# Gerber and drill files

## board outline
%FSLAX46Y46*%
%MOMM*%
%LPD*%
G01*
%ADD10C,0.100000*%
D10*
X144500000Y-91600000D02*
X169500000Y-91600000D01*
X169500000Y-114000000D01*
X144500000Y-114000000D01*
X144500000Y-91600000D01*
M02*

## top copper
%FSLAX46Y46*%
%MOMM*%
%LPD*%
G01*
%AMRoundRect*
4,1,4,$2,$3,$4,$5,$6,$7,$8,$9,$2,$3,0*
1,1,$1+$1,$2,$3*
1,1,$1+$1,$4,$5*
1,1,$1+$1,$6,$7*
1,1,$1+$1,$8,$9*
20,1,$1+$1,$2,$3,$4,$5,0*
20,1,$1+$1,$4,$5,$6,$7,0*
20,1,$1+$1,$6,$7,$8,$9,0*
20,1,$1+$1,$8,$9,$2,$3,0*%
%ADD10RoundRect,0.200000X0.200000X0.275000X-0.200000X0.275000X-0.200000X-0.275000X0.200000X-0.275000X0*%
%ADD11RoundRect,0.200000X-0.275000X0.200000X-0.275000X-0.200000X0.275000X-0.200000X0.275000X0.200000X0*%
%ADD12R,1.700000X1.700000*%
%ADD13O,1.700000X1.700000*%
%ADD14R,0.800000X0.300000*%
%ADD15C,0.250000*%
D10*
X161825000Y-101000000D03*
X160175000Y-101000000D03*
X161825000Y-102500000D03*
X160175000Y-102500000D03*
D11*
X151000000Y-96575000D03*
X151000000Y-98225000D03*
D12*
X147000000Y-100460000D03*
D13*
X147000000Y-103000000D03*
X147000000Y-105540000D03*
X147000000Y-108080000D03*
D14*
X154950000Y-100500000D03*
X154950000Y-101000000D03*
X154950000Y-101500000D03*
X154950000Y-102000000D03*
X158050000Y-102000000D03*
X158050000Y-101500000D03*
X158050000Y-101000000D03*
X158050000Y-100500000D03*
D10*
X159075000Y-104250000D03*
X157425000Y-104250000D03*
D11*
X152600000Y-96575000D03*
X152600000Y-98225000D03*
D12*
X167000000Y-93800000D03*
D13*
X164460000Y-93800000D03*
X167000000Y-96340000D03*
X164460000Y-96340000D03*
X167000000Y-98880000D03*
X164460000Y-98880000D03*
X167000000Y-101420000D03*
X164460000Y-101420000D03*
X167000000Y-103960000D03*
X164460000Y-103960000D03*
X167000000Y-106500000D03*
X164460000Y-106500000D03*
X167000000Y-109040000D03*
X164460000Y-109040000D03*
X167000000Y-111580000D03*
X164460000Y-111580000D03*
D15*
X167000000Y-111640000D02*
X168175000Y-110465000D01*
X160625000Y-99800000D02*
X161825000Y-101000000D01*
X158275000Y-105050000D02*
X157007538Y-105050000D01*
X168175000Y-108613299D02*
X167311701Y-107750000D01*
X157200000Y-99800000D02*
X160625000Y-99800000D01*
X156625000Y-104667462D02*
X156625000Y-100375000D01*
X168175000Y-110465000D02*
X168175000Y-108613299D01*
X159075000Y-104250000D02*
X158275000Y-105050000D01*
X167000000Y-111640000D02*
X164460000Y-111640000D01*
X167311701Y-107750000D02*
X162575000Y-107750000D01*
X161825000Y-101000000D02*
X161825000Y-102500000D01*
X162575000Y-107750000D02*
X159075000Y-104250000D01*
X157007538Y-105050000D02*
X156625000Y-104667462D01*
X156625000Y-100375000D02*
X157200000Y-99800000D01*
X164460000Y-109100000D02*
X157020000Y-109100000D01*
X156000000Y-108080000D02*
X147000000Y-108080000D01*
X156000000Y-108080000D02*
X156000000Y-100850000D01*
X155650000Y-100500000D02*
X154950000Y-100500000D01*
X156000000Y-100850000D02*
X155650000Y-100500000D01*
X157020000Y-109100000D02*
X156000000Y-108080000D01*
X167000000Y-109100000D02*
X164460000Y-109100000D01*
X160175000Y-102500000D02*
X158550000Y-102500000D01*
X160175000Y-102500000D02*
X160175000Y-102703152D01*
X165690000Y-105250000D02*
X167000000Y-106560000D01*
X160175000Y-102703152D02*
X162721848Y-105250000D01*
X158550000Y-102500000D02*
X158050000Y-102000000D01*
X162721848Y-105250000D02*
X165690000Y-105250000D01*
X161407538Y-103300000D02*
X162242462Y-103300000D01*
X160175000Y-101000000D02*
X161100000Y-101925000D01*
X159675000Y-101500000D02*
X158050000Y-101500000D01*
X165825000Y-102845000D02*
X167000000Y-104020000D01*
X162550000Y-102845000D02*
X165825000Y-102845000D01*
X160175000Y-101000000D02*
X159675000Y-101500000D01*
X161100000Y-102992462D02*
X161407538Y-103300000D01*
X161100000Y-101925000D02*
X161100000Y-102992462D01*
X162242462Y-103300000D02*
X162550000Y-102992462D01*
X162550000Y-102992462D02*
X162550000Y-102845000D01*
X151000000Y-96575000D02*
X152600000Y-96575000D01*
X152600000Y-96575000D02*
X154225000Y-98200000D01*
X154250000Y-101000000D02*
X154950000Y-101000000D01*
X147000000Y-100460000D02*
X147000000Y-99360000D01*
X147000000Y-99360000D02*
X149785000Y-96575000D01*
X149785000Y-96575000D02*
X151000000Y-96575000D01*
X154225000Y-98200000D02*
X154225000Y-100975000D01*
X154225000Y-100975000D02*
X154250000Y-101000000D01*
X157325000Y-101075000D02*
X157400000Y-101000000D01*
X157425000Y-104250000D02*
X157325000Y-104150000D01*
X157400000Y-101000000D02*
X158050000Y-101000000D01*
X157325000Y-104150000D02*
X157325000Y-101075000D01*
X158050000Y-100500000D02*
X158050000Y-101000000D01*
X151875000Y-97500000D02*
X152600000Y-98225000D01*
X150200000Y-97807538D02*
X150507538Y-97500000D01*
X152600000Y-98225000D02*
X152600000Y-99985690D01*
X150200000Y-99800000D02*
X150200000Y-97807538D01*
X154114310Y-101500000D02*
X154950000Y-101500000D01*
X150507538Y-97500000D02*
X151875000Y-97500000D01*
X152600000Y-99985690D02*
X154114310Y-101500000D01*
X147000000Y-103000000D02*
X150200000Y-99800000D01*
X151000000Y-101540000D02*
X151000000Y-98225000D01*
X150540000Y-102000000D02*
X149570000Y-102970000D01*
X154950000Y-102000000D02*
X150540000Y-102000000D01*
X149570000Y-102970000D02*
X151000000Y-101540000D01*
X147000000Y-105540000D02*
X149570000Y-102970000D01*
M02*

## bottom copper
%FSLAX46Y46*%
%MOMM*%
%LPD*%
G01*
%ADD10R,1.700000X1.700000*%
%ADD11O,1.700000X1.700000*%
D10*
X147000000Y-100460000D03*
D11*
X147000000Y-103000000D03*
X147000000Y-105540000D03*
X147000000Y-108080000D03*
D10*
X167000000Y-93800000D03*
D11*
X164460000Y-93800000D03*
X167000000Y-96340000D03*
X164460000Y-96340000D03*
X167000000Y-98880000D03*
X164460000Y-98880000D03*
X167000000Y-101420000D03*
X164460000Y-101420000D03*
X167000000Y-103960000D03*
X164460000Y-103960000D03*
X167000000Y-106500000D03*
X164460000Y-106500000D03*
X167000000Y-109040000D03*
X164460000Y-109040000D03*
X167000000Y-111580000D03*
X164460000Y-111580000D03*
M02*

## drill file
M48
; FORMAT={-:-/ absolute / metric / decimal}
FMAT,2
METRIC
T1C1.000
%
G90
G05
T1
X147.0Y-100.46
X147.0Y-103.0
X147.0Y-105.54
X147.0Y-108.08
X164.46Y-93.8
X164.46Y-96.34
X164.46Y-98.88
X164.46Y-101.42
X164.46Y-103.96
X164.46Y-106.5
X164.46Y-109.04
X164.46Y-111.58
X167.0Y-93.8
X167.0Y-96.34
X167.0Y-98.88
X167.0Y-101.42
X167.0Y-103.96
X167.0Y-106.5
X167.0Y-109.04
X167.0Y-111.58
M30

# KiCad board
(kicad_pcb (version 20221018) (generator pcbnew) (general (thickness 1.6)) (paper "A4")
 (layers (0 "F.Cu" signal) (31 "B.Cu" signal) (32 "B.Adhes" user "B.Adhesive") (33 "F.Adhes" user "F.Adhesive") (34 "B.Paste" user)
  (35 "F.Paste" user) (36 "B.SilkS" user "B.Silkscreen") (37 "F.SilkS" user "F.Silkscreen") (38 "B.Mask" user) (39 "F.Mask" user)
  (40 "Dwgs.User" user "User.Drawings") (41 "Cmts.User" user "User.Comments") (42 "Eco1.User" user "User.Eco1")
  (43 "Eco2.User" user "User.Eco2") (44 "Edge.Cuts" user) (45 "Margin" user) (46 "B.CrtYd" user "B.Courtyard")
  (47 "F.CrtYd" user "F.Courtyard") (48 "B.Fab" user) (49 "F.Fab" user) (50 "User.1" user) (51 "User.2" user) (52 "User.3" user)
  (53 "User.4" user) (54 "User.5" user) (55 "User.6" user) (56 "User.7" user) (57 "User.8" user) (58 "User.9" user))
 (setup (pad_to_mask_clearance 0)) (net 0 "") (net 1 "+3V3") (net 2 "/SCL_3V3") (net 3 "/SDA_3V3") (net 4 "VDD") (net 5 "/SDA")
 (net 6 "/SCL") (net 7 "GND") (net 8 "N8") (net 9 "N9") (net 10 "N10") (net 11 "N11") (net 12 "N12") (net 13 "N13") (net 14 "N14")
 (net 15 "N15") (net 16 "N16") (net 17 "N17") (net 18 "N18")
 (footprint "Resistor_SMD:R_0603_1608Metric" (layer "F.Cu") (at 161 101 180)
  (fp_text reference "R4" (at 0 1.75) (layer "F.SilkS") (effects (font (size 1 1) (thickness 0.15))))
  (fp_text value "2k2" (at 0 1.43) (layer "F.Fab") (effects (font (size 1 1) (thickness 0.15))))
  (pad "1" smd roundrect (at -0.825 0 180) (size 0.8 0.95) (layers "F.Cu" "F.Paste" "F.Mask") (roundrect_rratio 0.25) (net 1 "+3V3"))
  (pad "2" smd roundrect (at 0.825 0 180) (size 0.8 0.95) (layers "F.Cu" "F.Paste" "F.Mask") (roundrect_rratio 0.25) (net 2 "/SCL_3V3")))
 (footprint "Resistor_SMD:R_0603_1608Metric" (layer "F.Cu") (at 161 102.5 180)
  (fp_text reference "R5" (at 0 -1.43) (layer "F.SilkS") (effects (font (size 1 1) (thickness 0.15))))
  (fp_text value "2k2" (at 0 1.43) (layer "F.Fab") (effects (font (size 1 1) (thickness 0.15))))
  (pad "1" smd roundrect (at -0.825 0 180) (size 0.8 0.95) (layers "F.Cu" "F.Paste" "F.Mask") (roundrect_rratio 0.25) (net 1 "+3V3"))
  (pad "2" smd roundrect (at 0.825 0 180) (size 0.8 0.95) (layers "F.Cu" "F.Paste" "F.Mask") (roundrect_rratio 0.25) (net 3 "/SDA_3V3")))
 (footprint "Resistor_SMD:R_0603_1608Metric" (layer "F.Cu") (at 151 97.4 -90)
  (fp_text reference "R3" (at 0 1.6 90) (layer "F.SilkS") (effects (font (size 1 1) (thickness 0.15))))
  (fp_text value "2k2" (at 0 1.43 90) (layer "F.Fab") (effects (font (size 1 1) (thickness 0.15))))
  (pad "1" smd roundrect (at -0.825 0 270) (size 0.8 0.95) (layers "F.Cu" "F.Paste" "F.Mask") (roundrect_rratio 0.25) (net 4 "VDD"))
  (pad "2" smd roundrect (at 0.825 0 270) (size 0.8 0.95) (layers "F.Cu" "F.Paste" "F.Mask") (roundrect_rratio 0.25) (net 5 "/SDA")))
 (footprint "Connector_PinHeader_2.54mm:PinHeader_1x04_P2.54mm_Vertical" (layer "F.Cu") (at 147 100.46)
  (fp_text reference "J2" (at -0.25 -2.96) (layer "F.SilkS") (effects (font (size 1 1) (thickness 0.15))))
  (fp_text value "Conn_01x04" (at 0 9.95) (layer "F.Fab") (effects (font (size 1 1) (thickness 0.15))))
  (pad "1" thru_hole rect (at 0 0) (size 1.7 1.7) (drill 1) (layers "*.Cu" "*.Mask") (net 4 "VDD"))
  (pad "2" thru_hole oval (at 0 2.54) (size 1.7 1.7) (drill 1) (layers "*.Cu" "*.Mask") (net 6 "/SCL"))
  (pad "3" thru_hole oval (at 0 5.08) (size 1.7 1.7) (drill 1) (layers "*.Cu" "*.Mask") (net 5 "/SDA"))
  (pad "4" thru_hole oval (at 0 7.62) (size 1.7 1.7) (drill 1) (layers "*.Cu" "*.Mask") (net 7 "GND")))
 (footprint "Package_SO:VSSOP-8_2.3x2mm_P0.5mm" (layer "F.Cu") (at 156.5 101.25)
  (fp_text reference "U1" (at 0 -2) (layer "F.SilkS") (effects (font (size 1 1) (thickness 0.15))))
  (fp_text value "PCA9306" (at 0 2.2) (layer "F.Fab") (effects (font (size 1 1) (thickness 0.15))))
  (pad "1" smd rect (at -1.55 -0.75 270) (size 0.3 0.8) (layers "F.Cu" "F.Paste" "F.Mask") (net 7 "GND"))
  (pad "2" smd rect (at -1.55 -0.25 270) (size 0.3 0.8) (layers "F.Cu" "F.Paste" "F.Mask") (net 4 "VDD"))
  (pad "3" smd rect (at -1.55 0.25 270) (size 0.3 0.8) (layers "F.Cu" "F.Paste" "F.Mask") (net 6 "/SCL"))
  (pad "4" smd rect (at -1.55 0.75 270) (size 0.3 0.8) (layers "F.Cu" "F.Paste" "F.Mask") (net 5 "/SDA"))
  (pad "5" smd rect (at 1.55 0.75 270) (size 0.3 0.8) (layers "F.Cu" "F.Paste" "F.Mask") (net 3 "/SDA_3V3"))
  (pad "6" smd rect (at 1.55 0.25 270) (size 0.3 0.8) (layers "F.Cu" "F.Paste" "F.Mask") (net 2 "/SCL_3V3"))
  (pad "7" smd rect (at 1.55 -0.25 270) (size 0.3 0.8) (layers "F.Cu" "F.Paste" "F.Mask") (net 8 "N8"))
  (pad "8" smd rect (at 1.55 -0.75 270) (size 0.3 0.8) (layers "F.Cu" "F.Paste" "F.Mask") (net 8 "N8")))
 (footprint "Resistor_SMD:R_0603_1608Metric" (layer "F.Cu") (at 158.25 104.25 180)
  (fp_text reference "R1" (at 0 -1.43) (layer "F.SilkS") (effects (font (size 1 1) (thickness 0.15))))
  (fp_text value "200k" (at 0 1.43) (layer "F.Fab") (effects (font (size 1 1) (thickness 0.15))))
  (pad "1" smd roundrect (at -0.825 0 180) (size 0.8 0.95) (layers "F.Cu" "F.Paste" "F.Mask") (roundrect_rratio 0.25) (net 1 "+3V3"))
  (pad "2" smd roundrect (at 0.825 0 180) (size 0.8 0.95) (layers "F.Cu" "F.Paste" "F.Mask") (roundrect_rratio 0.25) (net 8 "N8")))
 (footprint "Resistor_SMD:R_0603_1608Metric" (layer "F.Cu") (at 152.6 97.4 -90)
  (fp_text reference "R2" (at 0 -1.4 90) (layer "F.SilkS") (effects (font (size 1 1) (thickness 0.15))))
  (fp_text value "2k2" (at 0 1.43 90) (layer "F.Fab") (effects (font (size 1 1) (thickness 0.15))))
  (pad "1" smd roundrect (at -0.825 0 270) (size 0.8 0.95) (layers "F.Cu" "F.Paste" "F.Mask") (roundrect_rratio 0.25) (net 4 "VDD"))
  (pad "2" smd roundrect (at 0.825 0 270) (size 0.8 0.95) (layers "F.Cu" "F.Paste" "F.Mask") (roundrect_rratio 0.25) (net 6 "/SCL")))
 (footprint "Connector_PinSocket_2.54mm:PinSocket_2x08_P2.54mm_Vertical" (layer "F.Cu") (at 167 93.8)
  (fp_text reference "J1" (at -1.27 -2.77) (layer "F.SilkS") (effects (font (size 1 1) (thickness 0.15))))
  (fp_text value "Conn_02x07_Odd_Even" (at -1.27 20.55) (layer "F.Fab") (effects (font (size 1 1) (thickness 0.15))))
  (pad "1" thru_hole rect (at 0 0) (size 1.7 1.7) (drill 1) (layers "*.Cu" "*.Mask") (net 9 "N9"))
  (pad "2" thru_hole oval (at -2.54 0) (size 1.7 1.7) (drill 1) (layers "*.Cu" "*.Mask") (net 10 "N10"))
  (pad "3" thru_hole oval (at 0 2.54) (size 1.7 1.7) (drill 1) (layers "*.Cu" "*.Mask") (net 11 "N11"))
  (pad "4" thru_hole oval (at -2.54 2.54) (size 1.7 1.7) (drill 1) (layers "*.Cu" "*.Mask") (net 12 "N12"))
  (pad "5" thru_hole oval (at 0 5.08) (size 1.7 1.7) (drill 1) (layers "*.Cu" "*.Mask") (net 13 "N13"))
  (pad "6" thru_hole oval (at -2.54 5.08) (size 1.7 1.7) (drill 1) (layers "*.Cu" "*.Mask") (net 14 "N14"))
  (pad "7" thru_hole oval (at 0 7.62) (size 1.7 1.7) (drill 1) (layers "*.Cu" "*.Mask") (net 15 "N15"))
  (pad "8" thru_hole oval (at -2.54 7.62) (size 1.7 1.7) (drill 1) (layers "*.Cu" "*.Mask") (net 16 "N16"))
  (pad "9" thru_hole oval (at 0 10.16) (size 1.7 1.7) (drill 1) (layers "*.Cu" "*.Mask") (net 2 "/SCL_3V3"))
  (pad "10" thru_hole oval (at -2.54 10.16) (size 1.7 1.7) (drill 1) (layers "*.Cu" "*.Mask") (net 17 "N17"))
  (pad "11" thru_hole oval (at 0 12.7) (size 1.7 1.7) (drill 1) (layers "*.Cu" "*.Mask") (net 3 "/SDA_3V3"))
  (pad "12" thru_hole oval (at -2.54 12.7) (size 1.7 1.7) (drill 1) (layers "*.Cu" "*.Mask") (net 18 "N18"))
  (pad "13" thru_hole oval (at 0 15.24) (size 1.7 1.7) (drill 1) (layers "*.Cu" "*.Mask") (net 7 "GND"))
  (pad "14" thru_hole oval (at -2.54 15.24) (size 1.7 1.7) (drill 1) (layers "*.Cu" "*.Mask") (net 7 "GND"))
  (pad "15" thru_hole oval (at 0 17.78) (size 1.7 1.7) (drill 1) (layers "*.Cu" "*.Mask") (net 1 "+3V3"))
  (pad "16" thru_hole oval (at -2.54 17.78) (size 1.7 1.7) (drill 1) (layers "*.Cu" "*.Mask") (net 1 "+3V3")))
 (gr_rect (start 144.5 91.6) (end 169.5 114) (stroke (width 0.1) (type default)) (fill none) (layer "Edge.Cuts"))
 (segment (start 167 111.64) (end 168.175 110.465) (width 0.25) (layer "F.Cu") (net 1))
 (segment (start 160.625 99.8) (end 161.825 101) (width 0.25) (layer "F.Cu") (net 1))
 (segment (start 158.275 105.05) (end 157.007538 105.05) (width 0.25) (layer "F.Cu") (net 1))
 (segment (start 168.175 108.613299) (end 167.311701 107.75) (width 0.25) (layer "F.Cu") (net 1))
 (segment (start 157.2 99.8) (end 160.625 99.8) (width 0.25) (layer "F.Cu") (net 1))
 (segment (start 156.625 104.667462) (end 156.625 100.375) (width 0.25) (layer "F.Cu") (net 1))
 (segment (start 168.175 110.465) (end 168.175 108.613299) (width 0.25) (layer "F.Cu") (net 1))
 (segment (start 159.075 104.25) (end 158.275 105.05) (width 0.25) (layer "F.Cu") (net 1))
 (segment (start 167 111.64) (end 164.46 111.64) (width 0.25) (layer "F.Cu") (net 1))
 (segment (start 167.311701 107.75) (end 162.575 107.75) (width 0.25) (layer "F.Cu") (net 1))
 (segment (start 161.825 101) (end 161.825 102.5) (width 0.25) (layer "F.Cu") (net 1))
 (segment (start 162.575 107.75) (end 159.075 104.25) (width 0.25) (layer "F.Cu") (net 1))
 (segment (start 157.007538 105.05) (end 156.625 104.667462) (width 0.25) (layer "F.Cu") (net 1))
 (segment (start 156.625 100.375) (end 157.2 99.8) (width 0.25) (layer "F.Cu") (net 1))
 (segment (start 164.46 109.1) (end 157.02 109.1) (width 0.25) (layer "F.Cu") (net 7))
 (segment (start 156 108.08) (end 147 108.08) (width 0.25) (layer "F.Cu") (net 7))
 (segment (start 156 108.08) (end 156 100.85) (width 0.25) (layer "F.Cu") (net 7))
 (segment (start 155.65 100.5) (end 154.95 100.5) (width 0.25) (layer "F.Cu") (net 7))
 (segment (start 156 100.85) (end 155.65 100.5) (width 0.25) (layer "F.Cu") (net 7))
 (segment (start 157.02 109.1) (end 156 108.08) (width 0.25) (layer "F.Cu") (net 7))
 (segment (start 167 109.1) (end 164.46 109.1) (width 0.25) (layer "F.Cu") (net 7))
 (segment (start 160.175 102.5) (end 158.55 102.5) (width 0.25) (layer "F.Cu") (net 3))
 (segment (start 160.175 102.5) (end 160.175 102.703152) (width 0.25) (layer "F.Cu") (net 3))
 (segment (start 165.69 105.25) (end 167 106.56) (width 0.25) (layer "F.Cu") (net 3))
 (segment (start 160.175 102.703152) (end 162.721848 105.25) (width 0.25) (layer "F.Cu") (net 3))
 (segment (start 158.55 102.5) (end 158.05 102) (width 0.25) (layer "F.Cu") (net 3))
 (segment (start 162.721848 105.25) (end 165.69 105.25) (width 0.25) (layer "F.Cu") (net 3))
 (segment (start 161.407538 103.3) (end 162.242462 103.3) (width 0.25) (layer "F.Cu") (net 2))
 (segment (start 160.175 101) (end 161.1 101.925) (width 0.25) (layer "F.Cu") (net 2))
 (segment (start 159.675 101.5) (end 158.05 101.5) (width 0.25) (layer "F.Cu") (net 2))
 (segment (start 165.825 102.845) (end 167 104.02) (width 0.25) (layer "F.Cu") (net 2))
 (segment (start 162.55 102.845) (end 165.825 102.845) (width 0.25) (layer "F.Cu") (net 2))
 (segment (start 160.175 101) (end 159.675 101.5) (width 0.25) (layer "F.Cu") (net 2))
 (segment (start 161.1 102.992462) (end 161.407538 103.3) (width 0.25) (layer "F.Cu") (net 2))
 (segment (start 161.1 101.925) (end 161.1 102.992462) (width 0.25) (layer "F.Cu") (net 2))
 (segment (start 162.242462 103.3) (end 162.55 102.992462) (width 0.25) (layer "F.Cu") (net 2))
 (segment (start 162.55 102.992462) (end 162.55 102.845) (width 0.25) (layer "F.Cu") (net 2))
 (segment (start 151 96.575) (end 152.6 96.575) (width 0.25) (layer "F.Cu") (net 4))
 (segment (start 152.6 96.575) (end 154.225 98.2) (width 0.25) (layer "F.Cu") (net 4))
 (segment (start 154.25 101) (end 154.95 101) (width 0.25) (layer "F.Cu") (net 4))
 (segment (start 147 100.46) (end 147 99.36) (width 0.25) (layer "F.Cu") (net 4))
 (segment (start 147 99.36) (end 149.785 96.575) (width 0.25) (layer "F.Cu") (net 4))
 (segment (start 149.785 96.575) (end 151 96.575) (width 0.25) (layer "F.Cu") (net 4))
 (segment (start 154.225 98.2) (end 154.225 100.975) (width 0.25) (layer "F.Cu") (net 4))
 (segment (start 154.225 100.975) (end 154.25 101) (width 0.25) (layer "F.Cu") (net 4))
 (segment (start 157.325 101.075) (end 157.4 101) (width 0.25) (layer "F.Cu") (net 8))
 (segment (start 157.425 104.25) (end 157.325 104.15) (width 0.25) (layer "F.Cu") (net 8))
 (segment (start 157.4 101) (end 158.05 101) (width 0.25) (layer "F.Cu") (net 8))
 (segment (start 157.325 104.15) (end 157.325 101.075) (width 0.25) (layer "F.Cu") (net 8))
 (segment (start 158.05 100.5) (end 158.05 101) (width 0.25) (layer "F.Cu") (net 8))
 (segment (start 151.875 97.5) (end 152.6 98.225) (width 0.25) (layer "F.Cu") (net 6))
 (segment (start 150.2 97.807538) (end 150.507538 97.5) (width 0.25) (layer "F.Cu") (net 6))
 (segment (start 152.6 98.225) (end 152.6 99.98569) (width 0.25) (layer "F.Cu") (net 6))
 (segment (start 150.2 99.8) (end 150.2 97.807538) (width 0.25) (layer "F.Cu") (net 6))
 (segment (start 154.11431 101.5) (end 154.95 101.5) (width 0.25) (layer "F.Cu") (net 6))
 (segment (start 150.507538 97.5) (end 151.875 97.5) (width 0.25) (layer "F.Cu") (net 6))
 (segment (start 152.6 99.98569) (end 154.11431 101.5) (width 0.25) (layer "F.Cu") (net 6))
 (segment (start 147 103) (end 150.2 99.8) (width 0.25) (layer "F.Cu") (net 6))
 (segment (start 151 101.54) (end 151 98.225) (width 0.25) (layer "F.Cu") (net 5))
 (segment (start 150.54 102) (end 149.57 102.97) (width 0.25) (layer "F.Cu") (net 5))
 (segment (start 154.95 102) (end 150.54 102) (width 0.25) (layer "F.Cu") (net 5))
 (segment (start 149.57 102.97) (end 151 101.54) (width 0.25) (layer "F.Cu") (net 5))
 (segment (start 147 105.54) (end 149.57 102.97) (width 0.25) (layer "F.Cu") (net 5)))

